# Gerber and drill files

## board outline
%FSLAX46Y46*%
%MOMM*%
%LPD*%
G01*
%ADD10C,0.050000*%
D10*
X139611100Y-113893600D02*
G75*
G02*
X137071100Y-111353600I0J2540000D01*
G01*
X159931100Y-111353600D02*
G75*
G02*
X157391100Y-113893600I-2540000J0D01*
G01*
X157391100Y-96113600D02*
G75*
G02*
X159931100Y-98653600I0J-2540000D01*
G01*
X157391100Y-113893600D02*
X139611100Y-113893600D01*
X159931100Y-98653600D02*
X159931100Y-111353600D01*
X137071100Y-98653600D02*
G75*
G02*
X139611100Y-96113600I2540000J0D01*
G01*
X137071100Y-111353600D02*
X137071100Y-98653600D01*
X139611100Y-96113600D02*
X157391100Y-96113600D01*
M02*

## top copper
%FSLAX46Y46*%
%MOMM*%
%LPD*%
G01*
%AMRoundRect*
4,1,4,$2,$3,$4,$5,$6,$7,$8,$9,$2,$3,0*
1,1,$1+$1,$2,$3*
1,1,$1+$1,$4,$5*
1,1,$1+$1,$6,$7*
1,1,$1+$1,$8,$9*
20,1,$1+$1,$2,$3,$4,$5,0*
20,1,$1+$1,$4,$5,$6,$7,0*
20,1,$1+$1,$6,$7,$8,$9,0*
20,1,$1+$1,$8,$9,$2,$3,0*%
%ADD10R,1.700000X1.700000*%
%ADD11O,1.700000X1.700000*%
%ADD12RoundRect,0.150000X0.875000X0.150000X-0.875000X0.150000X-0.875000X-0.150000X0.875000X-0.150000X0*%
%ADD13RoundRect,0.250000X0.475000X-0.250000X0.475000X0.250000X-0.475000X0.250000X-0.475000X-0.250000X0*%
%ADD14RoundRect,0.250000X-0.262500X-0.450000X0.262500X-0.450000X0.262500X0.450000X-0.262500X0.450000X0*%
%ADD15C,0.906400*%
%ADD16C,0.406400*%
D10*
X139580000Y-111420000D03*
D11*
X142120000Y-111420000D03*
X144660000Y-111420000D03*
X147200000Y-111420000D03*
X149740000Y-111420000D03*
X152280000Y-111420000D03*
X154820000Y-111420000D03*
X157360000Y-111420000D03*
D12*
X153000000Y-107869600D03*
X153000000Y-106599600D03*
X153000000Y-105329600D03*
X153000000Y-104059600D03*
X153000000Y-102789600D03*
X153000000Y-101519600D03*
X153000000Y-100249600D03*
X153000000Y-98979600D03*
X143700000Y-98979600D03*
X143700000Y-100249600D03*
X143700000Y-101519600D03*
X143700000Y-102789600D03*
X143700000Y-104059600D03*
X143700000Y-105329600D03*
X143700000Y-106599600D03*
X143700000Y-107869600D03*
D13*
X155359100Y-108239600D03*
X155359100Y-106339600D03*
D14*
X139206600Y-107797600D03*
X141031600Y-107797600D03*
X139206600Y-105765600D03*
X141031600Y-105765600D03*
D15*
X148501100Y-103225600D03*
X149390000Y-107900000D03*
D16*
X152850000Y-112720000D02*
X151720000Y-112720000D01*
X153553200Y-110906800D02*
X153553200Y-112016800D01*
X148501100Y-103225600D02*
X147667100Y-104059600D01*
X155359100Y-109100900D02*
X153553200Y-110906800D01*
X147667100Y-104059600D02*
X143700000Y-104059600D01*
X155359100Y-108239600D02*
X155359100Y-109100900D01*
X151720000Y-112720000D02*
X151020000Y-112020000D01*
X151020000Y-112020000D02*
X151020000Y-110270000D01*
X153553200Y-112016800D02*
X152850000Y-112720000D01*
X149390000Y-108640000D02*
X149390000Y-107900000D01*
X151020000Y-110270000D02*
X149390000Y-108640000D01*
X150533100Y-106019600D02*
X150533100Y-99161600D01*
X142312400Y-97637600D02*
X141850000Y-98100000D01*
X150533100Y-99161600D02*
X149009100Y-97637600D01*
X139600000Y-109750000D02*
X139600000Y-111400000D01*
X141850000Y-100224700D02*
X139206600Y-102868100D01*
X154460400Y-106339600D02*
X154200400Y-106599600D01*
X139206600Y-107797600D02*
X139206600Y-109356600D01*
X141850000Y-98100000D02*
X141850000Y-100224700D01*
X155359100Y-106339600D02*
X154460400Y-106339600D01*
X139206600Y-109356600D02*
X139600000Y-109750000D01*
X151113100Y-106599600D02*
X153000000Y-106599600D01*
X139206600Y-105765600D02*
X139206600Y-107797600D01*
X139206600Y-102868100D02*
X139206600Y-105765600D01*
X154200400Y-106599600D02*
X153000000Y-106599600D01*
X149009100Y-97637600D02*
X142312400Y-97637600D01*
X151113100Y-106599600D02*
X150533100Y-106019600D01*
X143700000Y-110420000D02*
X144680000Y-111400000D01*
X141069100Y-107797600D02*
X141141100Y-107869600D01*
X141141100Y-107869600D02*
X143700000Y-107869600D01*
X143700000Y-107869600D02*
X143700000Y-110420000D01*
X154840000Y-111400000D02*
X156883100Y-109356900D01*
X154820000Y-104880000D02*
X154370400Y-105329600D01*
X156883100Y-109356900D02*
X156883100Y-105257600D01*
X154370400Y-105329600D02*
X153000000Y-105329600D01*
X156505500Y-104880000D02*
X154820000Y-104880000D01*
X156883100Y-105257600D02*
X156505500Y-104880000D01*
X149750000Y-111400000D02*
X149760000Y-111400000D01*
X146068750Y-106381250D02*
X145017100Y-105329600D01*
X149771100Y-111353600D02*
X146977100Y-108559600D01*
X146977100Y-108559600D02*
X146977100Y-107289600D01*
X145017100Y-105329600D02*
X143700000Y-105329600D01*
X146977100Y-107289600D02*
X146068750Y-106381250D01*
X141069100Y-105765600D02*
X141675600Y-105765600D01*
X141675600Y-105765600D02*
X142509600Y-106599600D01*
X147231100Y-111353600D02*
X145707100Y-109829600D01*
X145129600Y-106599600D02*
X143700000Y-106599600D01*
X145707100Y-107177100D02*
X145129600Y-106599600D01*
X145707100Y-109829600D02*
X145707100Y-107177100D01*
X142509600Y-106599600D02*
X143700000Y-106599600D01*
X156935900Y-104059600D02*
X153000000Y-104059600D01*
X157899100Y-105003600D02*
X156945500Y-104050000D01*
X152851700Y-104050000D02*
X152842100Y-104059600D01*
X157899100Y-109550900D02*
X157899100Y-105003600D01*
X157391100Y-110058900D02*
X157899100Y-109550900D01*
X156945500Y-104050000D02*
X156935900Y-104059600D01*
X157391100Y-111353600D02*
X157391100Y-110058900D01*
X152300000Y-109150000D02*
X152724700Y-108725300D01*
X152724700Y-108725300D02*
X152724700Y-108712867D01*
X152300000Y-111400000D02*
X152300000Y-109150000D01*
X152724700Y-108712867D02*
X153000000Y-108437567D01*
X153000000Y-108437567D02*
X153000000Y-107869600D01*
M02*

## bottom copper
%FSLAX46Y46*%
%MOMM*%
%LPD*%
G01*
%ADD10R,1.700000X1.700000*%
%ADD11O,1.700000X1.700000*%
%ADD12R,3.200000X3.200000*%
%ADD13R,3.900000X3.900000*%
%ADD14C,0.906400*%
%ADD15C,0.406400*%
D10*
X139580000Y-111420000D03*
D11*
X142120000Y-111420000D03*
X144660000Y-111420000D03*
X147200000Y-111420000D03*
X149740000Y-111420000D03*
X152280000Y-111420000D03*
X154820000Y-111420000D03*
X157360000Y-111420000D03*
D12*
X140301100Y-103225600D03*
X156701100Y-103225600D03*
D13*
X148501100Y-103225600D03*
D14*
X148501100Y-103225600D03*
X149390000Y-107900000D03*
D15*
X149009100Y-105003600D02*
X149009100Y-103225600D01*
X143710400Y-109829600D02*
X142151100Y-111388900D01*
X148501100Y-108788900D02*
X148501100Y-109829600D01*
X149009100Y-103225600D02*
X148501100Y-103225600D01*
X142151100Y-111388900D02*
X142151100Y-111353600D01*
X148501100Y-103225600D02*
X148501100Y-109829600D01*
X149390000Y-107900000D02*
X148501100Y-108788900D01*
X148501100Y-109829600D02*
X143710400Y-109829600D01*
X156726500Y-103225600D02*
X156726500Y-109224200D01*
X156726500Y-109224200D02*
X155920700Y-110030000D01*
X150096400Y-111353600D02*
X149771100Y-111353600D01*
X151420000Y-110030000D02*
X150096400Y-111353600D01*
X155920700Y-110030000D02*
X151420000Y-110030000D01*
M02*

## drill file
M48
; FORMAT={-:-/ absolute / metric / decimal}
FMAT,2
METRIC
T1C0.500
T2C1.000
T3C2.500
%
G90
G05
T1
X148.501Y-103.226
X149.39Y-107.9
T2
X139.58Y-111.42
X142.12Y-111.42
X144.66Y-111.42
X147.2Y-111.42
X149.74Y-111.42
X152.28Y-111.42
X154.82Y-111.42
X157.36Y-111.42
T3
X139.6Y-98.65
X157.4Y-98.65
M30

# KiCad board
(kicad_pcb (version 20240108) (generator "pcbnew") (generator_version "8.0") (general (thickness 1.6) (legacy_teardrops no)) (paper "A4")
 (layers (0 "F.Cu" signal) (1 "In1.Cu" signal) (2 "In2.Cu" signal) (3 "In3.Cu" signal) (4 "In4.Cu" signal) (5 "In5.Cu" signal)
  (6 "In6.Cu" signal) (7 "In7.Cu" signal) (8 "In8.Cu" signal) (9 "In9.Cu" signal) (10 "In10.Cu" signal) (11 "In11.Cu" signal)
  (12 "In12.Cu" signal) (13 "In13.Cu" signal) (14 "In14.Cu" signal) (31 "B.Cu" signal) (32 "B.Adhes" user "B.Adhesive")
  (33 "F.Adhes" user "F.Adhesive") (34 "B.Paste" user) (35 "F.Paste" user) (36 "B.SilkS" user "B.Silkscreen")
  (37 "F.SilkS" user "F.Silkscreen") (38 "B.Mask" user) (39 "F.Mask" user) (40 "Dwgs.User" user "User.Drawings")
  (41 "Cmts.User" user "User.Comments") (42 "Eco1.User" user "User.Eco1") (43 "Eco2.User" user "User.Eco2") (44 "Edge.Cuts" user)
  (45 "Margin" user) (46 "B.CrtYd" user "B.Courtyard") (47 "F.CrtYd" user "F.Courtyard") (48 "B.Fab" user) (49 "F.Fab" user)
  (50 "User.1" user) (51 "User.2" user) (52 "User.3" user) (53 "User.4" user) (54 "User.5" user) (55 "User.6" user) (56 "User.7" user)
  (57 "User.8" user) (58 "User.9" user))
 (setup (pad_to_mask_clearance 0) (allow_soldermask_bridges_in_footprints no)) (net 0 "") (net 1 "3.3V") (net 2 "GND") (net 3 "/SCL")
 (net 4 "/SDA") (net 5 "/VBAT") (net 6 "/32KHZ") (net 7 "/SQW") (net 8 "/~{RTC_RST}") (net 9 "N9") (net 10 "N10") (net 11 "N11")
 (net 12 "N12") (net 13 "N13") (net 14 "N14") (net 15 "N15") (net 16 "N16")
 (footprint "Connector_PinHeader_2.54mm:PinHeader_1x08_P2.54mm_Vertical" (layer "F.Cu") (at 139.58 111.42 90)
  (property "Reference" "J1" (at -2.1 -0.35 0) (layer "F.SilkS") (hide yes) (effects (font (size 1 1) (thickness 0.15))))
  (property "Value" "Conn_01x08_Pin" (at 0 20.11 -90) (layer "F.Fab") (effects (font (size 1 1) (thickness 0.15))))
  (pad "1" thru_hole rect (at 0 0 90) (size 1.7 1.7) (drill 1) (layers "*.Cu" "*.Mask") (remove_unused_layers no) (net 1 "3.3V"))
  (pad "2" thru_hole oval (at 0 2.54 90) (size 1.7 1.7) (drill 1) (layers "*.Cu" "*.Mask") (remove_unused_layers no) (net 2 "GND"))
  (pad "3" thru_hole oval (at 0 5.08 90) (size 1.7 1.7) (drill 1) (layers "*.Cu" "*.Mask") (remove_unused_layers no) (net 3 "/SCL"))
  (pad "4" thru_hole oval (at 0 7.62 90) (size 1.7 1.7) (drill 1) (layers "*.Cu" "*.Mask") (remove_unused_layers no) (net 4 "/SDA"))
  (pad "5" thru_hole oval (at 0 10.16 90) (size 1.7 1.7) (drill 1) (layers "*.Cu" "*.Mask") (remove_unused_layers no) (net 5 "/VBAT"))
  (pad "6" thru_hole oval (at 0 12.7 90) (size 1.7 1.7) (drill 1) (layers "*.Cu" "*.Mask") (remove_unused_layers no) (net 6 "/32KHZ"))
  (pad "7" thru_hole oval (at 0 15.24 90) (size 1.7 1.7) (drill 1) (layers "*.Cu" "*.Mask") (remove_unused_layers no) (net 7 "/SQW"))
  (pad "8" thru_hole oval (at 0 17.78 90) (size 1.7 1.7) (drill 1) (layers "*.Cu" "*.Mask") (remove_unused_layers no) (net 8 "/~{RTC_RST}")))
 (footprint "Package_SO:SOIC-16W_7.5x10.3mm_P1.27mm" (layer "F.Cu") (at 148.35 103.4246 180)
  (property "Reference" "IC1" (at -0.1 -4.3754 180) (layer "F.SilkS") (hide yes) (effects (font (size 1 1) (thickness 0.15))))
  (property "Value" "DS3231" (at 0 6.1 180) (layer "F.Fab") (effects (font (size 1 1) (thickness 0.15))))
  (pad "1" smd roundrect (at -4.65 -4.445 180) (size 2.05 0.6) (layers "F.Cu" "F.Paste" "F.Mask") (roundrect_rratio 0.25) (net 6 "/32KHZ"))
  (pad "2" smd roundrect (at -4.65 -3.175 180) (size 2.05 0.6) (layers "F.Cu" "F.Paste" "F.Mask") (roundrect_rratio 0.25) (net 1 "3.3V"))
  (pad "3" smd roundrect (at -4.65 -1.905 180) (size 2.05 0.6) (layers "F.Cu" "F.Paste" "F.Mask") (roundrect_rratio 0.25) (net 7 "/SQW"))
  (pad "4" smd roundrect (at -4.65 -0.635 180) (size 2.05 0.6) (layers "F.Cu" "F.Paste" "F.Mask") (roundrect_rratio 0.25)
   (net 8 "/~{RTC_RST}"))
  (pad "5" smd roundrect (at -4.65 0.635 180) (size 2.05 0.6) (layers "F.Cu" "F.Paste" "F.Mask") (roundrect_rratio 0.25) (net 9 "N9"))
  (pad "6" smd roundrect (at -4.65 1.905 180) (size 2.05 0.6) (layers "F.Cu" "F.Paste" "F.Mask") (roundrect_rratio 0.25) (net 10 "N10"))
  (pad "7" smd roundrect (at -4.65 3.175 180) (size 2.05 0.6) (layers "F.Cu" "F.Paste" "F.Mask") (roundrect_rratio 0.25) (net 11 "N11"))
  (pad "8" smd roundrect (at -4.65 4.445 180) (size 2.05 0.6) (layers "F.Cu" "F.Paste" "F.Mask") (roundrect_rratio 0.25) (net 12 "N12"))
  (pad "9" smd roundrect (at 4.65 4.445 180) (size 2.05 0.6) (layers "F.Cu" "F.Paste" "F.Mask") (roundrect_rratio 0.25) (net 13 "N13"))
  (pad "10" smd roundrect (at 4.65 3.175 180) (size 2.05 0.6) (layers "F.Cu" "F.Paste" "F.Mask") (roundrect_rratio 0.25) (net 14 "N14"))
  (pad "11" smd roundrect (at 4.65 1.905 180) (size 2.05 0.6) (layers "F.Cu" "F.Paste" "F.Mask") (roundrect_rratio 0.25) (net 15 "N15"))
  (pad "12" smd roundrect (at 4.65 0.635 180) (size 2.05 0.6) (layers "F.Cu" "F.Paste" "F.Mask") (roundrect_rratio 0.25) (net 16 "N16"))
  (pad "13" smd roundrect (at 4.65 -0.635 180) (size 2.05 0.6) (layers "F.Cu" "F.Paste" "F.Mask") (roundrect_rratio 0.25) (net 2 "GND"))
  (pad "14" smd roundrect (at 4.65 -1.905 180) (size 2.05 0.6) (layers "F.Cu" "F.Paste" "F.Mask") (roundrect_rratio 0.25) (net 5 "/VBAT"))
  (pad "15" smd roundrect (at 4.65 -3.175 180) (size 2.05 0.6) (layers "F.Cu" "F.Paste" "F.Mask") (roundrect_rratio 0.25) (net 4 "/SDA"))
  (pad "16" smd roundrect (at 4.65 -4.445 180) (size 2.05 0.6) (layers "F.Cu" "F.Paste" "F.Mask") (roundrect_rratio 0.25) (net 3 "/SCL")))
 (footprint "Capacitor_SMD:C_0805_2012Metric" (layer "F.Cu") (at 155.3591 107.2896 90)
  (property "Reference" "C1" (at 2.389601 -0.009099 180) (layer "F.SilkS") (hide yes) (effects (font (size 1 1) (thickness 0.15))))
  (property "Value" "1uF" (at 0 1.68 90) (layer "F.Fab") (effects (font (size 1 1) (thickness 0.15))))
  (pad "1" smd roundrect (at -0.95 0 90) (size 1 1.45) (layers "F.Cu" "F.Paste" "F.Mask") (roundrect_rratio 0.25) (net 2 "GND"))
  (pad "2" smd roundrect (at 0.95 0 90) (size 1 1.45) (layers "F.Cu" "F.Paste" "F.Mask") (roundrect_rratio 0.25) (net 1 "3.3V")))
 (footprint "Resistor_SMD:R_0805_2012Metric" (layer "F.Cu") (at 140.1191 107.7976)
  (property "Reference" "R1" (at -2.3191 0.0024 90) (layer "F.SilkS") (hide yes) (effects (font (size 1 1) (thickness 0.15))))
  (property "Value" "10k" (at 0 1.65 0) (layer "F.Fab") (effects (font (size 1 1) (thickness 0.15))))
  (pad "1" smd roundrect (at -0.9125 0) (size 1.025 1.4) (layers "F.Cu" "F.Paste" "F.Mask") (roundrect_rratio 0.243902) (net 1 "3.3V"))
  (pad "2" smd roundrect (at 0.9125 0) (size 1.025 1.4) (layers "F.Cu" "F.Paste" "F.Mask") (roundrect_rratio 0.243902) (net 3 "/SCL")))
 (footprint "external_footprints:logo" (layer "F.Cu") (at 157 102.74)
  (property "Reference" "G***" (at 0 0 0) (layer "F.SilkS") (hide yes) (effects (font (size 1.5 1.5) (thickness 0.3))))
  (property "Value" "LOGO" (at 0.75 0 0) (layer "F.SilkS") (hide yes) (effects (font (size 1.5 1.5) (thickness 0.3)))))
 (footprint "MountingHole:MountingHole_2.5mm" (layer "F.Cu") (at 157.4 98.65)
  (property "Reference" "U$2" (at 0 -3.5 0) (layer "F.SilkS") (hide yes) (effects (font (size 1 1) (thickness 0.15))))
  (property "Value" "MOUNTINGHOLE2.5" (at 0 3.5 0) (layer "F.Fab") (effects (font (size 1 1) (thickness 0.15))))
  (pad "" np_thru_hole circle (at 0 0) (size 2.5 2.5) (drill 2.5) (layers "*.Cu" "*.Mask")))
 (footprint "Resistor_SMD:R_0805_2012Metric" (layer "F.Cu") (at 140.1191 105.7656)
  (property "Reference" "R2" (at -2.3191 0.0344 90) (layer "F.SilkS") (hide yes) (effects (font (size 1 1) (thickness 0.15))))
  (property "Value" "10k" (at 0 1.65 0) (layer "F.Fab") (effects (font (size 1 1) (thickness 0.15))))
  (pad "1" smd roundrect (at -0.9125 0) (size 1.025 1.4) (layers "F.Cu" "F.Paste" "F.Mask") (roundrect_rratio 0.243902) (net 1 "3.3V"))
  (pad "2" smd roundrect (at 0.9125 0) (size 1.025 1.4) (layers "F.Cu" "F.Paste" "F.Mask") (roundrect_rratio 0.243902) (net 4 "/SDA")))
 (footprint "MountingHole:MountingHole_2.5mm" (layer "F.Cu") (at 139.6 98.65)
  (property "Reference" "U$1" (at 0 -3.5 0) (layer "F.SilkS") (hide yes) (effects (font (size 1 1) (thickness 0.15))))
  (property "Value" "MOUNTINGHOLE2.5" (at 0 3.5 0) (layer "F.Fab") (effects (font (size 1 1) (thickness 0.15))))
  (pad "" np_thru_hole circle (at 0 0) (size 2.5 2.5) (drill 2.5) (layers "*.Cu" "*.Mask")))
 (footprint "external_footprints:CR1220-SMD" (layer "B.Cu") (at 148.5011 103.2256 180)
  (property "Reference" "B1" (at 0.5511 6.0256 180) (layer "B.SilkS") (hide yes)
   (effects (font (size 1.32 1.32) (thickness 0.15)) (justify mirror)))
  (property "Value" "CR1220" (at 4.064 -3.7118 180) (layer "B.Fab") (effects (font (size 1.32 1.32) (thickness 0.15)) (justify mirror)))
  (pad "" smd rect (at 8.2 0 180) (size 3.2 3.2) (layers "B.Cu" "B.Paste" "B.Mask") (solder_mask_margin 0.102))
  (pad "1" smd rect (at -8.2 0 180) (size 3.2 3.2) (layers "B.Cu" "B.Paste" "B.Mask") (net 5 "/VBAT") (solder_mask_margin 0.102))
  (pad "2" smd rect (at 0 0 180) (size 3.9 3.9) (layers "B.Cu" "B.Paste" "B.Mask") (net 2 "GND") (solder_mask_margin 0.102)))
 (gr_arc (start 139.6111 113.8936) (mid 137.815049 113.149651) (end 137.0711 111.3536) (stroke (width 0.05) (type solid))
  (layer "Edge.Cuts"))
 (gr_arc (start 159.9311 111.3536) (mid 159.187151 113.149651) (end 157.3911 113.8936) (stroke (width 0.05) (type solid))
  (layer "Edge.Cuts"))
 (gr_arc (start 157.3911 96.1136) (mid 159.187151 96.857549) (end 159.9311 98.6536) (stroke (width 0.05) (type solid)) (layer "Edge.Cuts"))
 (gr_line (start 157.3911 113.8936) (end 139.6111 113.8936) (stroke (width 0.05) (type solid)) (layer "Edge.Cuts"))
 (gr_line (start 159.9311 98.6536) (end 159.9311 111.3536) (stroke (width 0.05) (type solid)) (layer "Edge.Cuts"))
 (gr_arc (start 137.0711 98.6536) (mid 137.815049 96.857549) (end 139.6111 96.1136) (stroke (width 0.05) (type solid)) (layer "Edge.Cuts"))
 (gr_line (start 137.0711 111.3536) (end 137.0711 98.6536) (stroke (width 0.05) (type solid)) (layer "Edge.Cuts"))
 (gr_line (start 139.6111 96.1136) (end 157.3911 96.1136) (stroke (width 0.05) (type solid)) (layer "Edge.Cuts"))
 (segment (start 152.85 112.72) (end 151.72 112.72) (width 0.4064) (layer "F.Cu") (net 2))
 (segment (start 153.5532 110.9068) (end 153.5532 112.0168) (width 0.4064) (layer "F.Cu") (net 2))
 (segment (start 148.5011 103.2256) (end 147.6671 104.0596) (width 0.4064) (layer "F.Cu") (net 2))
 (segment (start 155.3591 109.1009) (end 153.5532 110.9068) (width 0.4064) (layer "F.Cu") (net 2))
 (segment (start 147.6671 104.0596) (end 143.7 104.0596) (width 0.4064) (layer "F.Cu") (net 2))
 (segment (start 155.3591 108.2396) (end 155.3591 109.1009) (width 0.4064) (layer "F.Cu") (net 2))
 (segment (start 151.72 112.72) (end 151.02 112.02) (width 0.4064) (layer "F.Cu") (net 2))
 (segment (start 151.02 112.02) (end 151.02 110.27) (width 0.4064) (layer "F.Cu") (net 2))
 (segment (start 153.5532 112.0168) (end 152.85 112.72) (width 0.4064) (layer "F.Cu") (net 2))
 (segment (start 149.39 108.64) (end 149.39 107.9) (width 0.4064) (layer "F.Cu") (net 2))
 (segment (start 151.02 110.27) (end 149.39 108.64) (width 0.4064) (layer "F.Cu") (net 2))
 (via (at 148.5011 103.2256) (size 0.9064) (drill 0.5) (layers "F.Cu" "B.Cu") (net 2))
 (via (at 149.39 107.9) (size 0.9064) (drill 0.5) (layers "F.Cu" "B.Cu") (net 2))
 (segment (start 149.0091 105.0036) (end 149.0091 103.2256) (width 0.4064) (layer "B.Cu") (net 2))
 (segment (start 143.7104 109.8296) (end 142.1511 111.3889) (width 0.4064) (layer "B.Cu") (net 2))
 (segment (start 148.5011 108.7889) (end 148.5011 109.8296) (width 0.4064) (layer "B.Cu") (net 2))
 (segment (start 149.0091 103.2256) (end 148.5011 103.2256) (width 0.4064) (layer "B.Cu") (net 2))
 (segment (start 142.1511 111.3889) (end 142.1511 111.3536) (width 0.4064) (layer "B.Cu") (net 2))
 (segment (start 148.5011 103.2256) (end 148.5011 109.8296) (width 0.4064) (layer "B.Cu") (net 2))
 (segment (start 149.39 107.9) (end 148.5011 108.7889) (width 0.4064) (layer "B.Cu") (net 2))
 (segment (start 148.5011 109.8296) (end 143.7104 109.8296) (width 0.4064) (layer "B.Cu") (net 2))
 (segment (start 150.5331 106.0196) (end 150.5331 99.1616) (width 0.4064) (layer "F.Cu") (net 1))
 (segment (start 142.3124 97.6376) (end 141.85 98.1) (width 0.4064) (layer "F.Cu") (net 1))
 (segment (start 150.5331 99.1616) (end 149.0091 97.6376) (width 0.4064) (layer "F.Cu") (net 1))
 (segment (start 139.6 109.75) (end 139.6 111.4) (width 0.4064) (layer "F.Cu") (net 1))
 (segment (start 141.85 100.2247) (end 139.2066 102.8681) (width 0.4064) (layer "F.Cu") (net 1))
 (segment (start 154.4604 106.3396) (end 154.2004 106.5996) (width 0.4064) (layer "F.Cu") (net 1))
 (segment (start 139.2066 107.7976) (end 139.2066 109.3566) (width 0.4064) (layer "F.Cu") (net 1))
 (segment (start 141.85 98.1) (end 141.85 100.2247) (width 0.4064) (layer "F.Cu") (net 1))
 (segment (start 155.3591 106.3396) (end 154.4604 106.3396) (width 0.4064) (layer "F.Cu") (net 1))
 (segment (start 139.2066 109.3566) (end 139.6 109.75) (width 0.4064) (layer "F.Cu") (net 1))
 (segment (start 151.1131 106.5996) (end 153 106.5996) (width 0.4064) (layer "F.Cu") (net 1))
 (segment (start 139.2066 105.7656) (end 139.2066 107.7976) (width 0.4064) (layer "F.Cu") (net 1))
 (segment (start 139.2066 102.8681) (end 139.2066 105.7656) (width 0.4064) (layer "F.Cu") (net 1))
 (segment (start 154.2004 106.5996) (end 153 106.5996) (width 0.4064) (layer "F.Cu") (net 1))
 (segment (start 149.0091 97.6376) (end 142.3124 97.6376) (width 0.4064) (layer "F.Cu") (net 1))
 (segment (start 151.1131 106.5996) (end 150.5331 106.0196) (width 0.4064) (layer "F.Cu") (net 1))
 (segment (start 143.7 110.42) (end 144.68 111.4) (width 0.4064) (layer "F.Cu") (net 3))
 (segment (start 141.0691 107.7976) (end 141.1411 107.8696) (width 0.4064) (layer "F.Cu") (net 3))
 (segment (start 141.1411 107.8696) (end 143.7 107.8696) (width 0.4064) (layer "F.Cu") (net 3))
 (segment (start 143.7 107.8696) (end 143.7 110.42) (width 0.4064) (layer "F.Cu") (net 3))
 (segment (start 154.84 111.4) (end 156.8831 109.3569) (width 0.4064) (layer "F.Cu") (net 7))
 (segment (start 154.82 104.88) (end 154.3704 105.3296) (width 0.4064) (layer "F.Cu") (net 7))
 (segment (start 156.8831 109.3569) (end 156.8831 105.2576) (width 0.4064) (layer "F.Cu") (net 7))
 (segment (start 154.3704 105.3296) (end 153 105.3296) (width 0.4064) (layer "F.Cu") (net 7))
 (segment (start 156.5055 104.88) (end 154.82 104.88) (width 0.4064) (layer "F.Cu") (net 7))
 (segment (start 156.8831 105.2576) (end 156.5055 104.88) (width 0.4064) (layer "F.Cu") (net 7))
 (segment (start 149.75 111.4) (end 149.76 111.4) (width 0.4064) (layer "F.Cu") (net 5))
 (segment (start 146.06875 106.38125) (end 145.0171 105.3296) (width 0.4064) (layer "F.Cu") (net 5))
 (segment (start 149.7711 111.3536) (end 146.9771 108.5596) (width 0.4064) (layer "F.Cu") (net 5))
 (segment (start 146.9771 108.5596) (end 146.9771 107.2896) (width 0.4064) (layer "F.Cu") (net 5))
 (segment (start 145.0171 105.3296) (end 143.7 105.3296) (width 0.4064) (layer "F.Cu") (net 5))
 (segment (start 146.9771 107.2896) (end 146.06875 106.38125) (width 0.4064) (layer "F.Cu") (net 5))
 (segment (start 156.7265 103.2256) (end 156.7265 109.2242) (width 0.4064) (layer "B.Cu") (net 5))
 (segment (start 156.7265 109.2242) (end 155.9207 110.03) (width 0.4064) (layer "B.Cu") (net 5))
 (segment (start 150.0964 111.3536) (end 149.7711 111.3536) (width 0.4064) (layer "B.Cu") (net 5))
 (segment (start 151.42 110.03) (end 150.0964 111.3536) (width 0.4064) (layer "B.Cu") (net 5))
 (segment (start 155.9207 110.03) (end 151.42 110.03) (width 0.4064) (layer "B.Cu") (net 5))
 (segment (start 141.0691 105.7656) (end 141.6756 105.7656) (width 0.4064) (layer "F.Cu") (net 4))
 (segment (start 141.6756 105.7656) (end 142.5096 106.5996) (width 0.4064) (layer "F.Cu") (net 4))
 (segment (start 147.2311 111.3536) (end 145.7071 109.8296) (width 0.4064) (layer "F.Cu") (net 4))
 (segment (start 145.1296 106.5996) (end 143.7 106.5996) (width 0.4064) (layer "F.Cu") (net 4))
 (segment (start 145.7071 107.1771) (end 145.1296 106.5996) (width 0.4064) (layer "F.Cu") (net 4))
 (segment (start 145.7071 109.8296) (end 145.7071 107.1771) (width 0.4064) (layer "F.Cu") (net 4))
 (segment (start 142.5096 106.5996) (end 143.7 106.5996) (width 0.4064) (layer "F.Cu") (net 4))
 (segment (start 156.9359 104.0596) (end 153 104.0596) (width 0.4064) (layer "F.Cu") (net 8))
 (segment (start 157.8991 105.0036) (end 156.9455 104.05) (width 0.4064) (layer "F.Cu") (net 8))
 (segment (start 152.8517 104.05) (end 152.8421 104.0596) (width 0.4064) (layer "F.Cu") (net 8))
 (segment (start 157.8991 109.5509) (end 157.8991 105.0036) (width 0.4064) (layer "F.Cu") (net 8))
 (segment (start 157.3911 110.0589) (end 157.8991 109.5509) (width 0.4064) (layer "F.Cu") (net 8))
 (segment (start 156.9455 104.05) (end 156.9359 104.0596) (width 0.4064) (layer "F.Cu") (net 8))
 (segment (start 157.3911 111.3536) (end 157.3911 110.0589) (width 0.4064) (layer "F.Cu") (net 8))
 (segment (start 152.3 109.15) (end 152.7247 108.7253) (width 0.4064) (layer "F.Cu") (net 6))
 (segment (start 152.7247 108.7253) (end 152.7247 108.712867) (width 0.4064) (layer "F.Cu") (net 6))
 (segment (start 152.3 111.4) (end 152.3 109.15) (width 0.4064) (layer "F.Cu") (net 6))
 (segment (start 152.7247 108.712867) (end 153 108.437567) (width 0.4064) (layer "F.Cu") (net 6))
 (segment (start 153 108.437567) (end 153 107.8696) (width 0.4064) (layer "F.Cu") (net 6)))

